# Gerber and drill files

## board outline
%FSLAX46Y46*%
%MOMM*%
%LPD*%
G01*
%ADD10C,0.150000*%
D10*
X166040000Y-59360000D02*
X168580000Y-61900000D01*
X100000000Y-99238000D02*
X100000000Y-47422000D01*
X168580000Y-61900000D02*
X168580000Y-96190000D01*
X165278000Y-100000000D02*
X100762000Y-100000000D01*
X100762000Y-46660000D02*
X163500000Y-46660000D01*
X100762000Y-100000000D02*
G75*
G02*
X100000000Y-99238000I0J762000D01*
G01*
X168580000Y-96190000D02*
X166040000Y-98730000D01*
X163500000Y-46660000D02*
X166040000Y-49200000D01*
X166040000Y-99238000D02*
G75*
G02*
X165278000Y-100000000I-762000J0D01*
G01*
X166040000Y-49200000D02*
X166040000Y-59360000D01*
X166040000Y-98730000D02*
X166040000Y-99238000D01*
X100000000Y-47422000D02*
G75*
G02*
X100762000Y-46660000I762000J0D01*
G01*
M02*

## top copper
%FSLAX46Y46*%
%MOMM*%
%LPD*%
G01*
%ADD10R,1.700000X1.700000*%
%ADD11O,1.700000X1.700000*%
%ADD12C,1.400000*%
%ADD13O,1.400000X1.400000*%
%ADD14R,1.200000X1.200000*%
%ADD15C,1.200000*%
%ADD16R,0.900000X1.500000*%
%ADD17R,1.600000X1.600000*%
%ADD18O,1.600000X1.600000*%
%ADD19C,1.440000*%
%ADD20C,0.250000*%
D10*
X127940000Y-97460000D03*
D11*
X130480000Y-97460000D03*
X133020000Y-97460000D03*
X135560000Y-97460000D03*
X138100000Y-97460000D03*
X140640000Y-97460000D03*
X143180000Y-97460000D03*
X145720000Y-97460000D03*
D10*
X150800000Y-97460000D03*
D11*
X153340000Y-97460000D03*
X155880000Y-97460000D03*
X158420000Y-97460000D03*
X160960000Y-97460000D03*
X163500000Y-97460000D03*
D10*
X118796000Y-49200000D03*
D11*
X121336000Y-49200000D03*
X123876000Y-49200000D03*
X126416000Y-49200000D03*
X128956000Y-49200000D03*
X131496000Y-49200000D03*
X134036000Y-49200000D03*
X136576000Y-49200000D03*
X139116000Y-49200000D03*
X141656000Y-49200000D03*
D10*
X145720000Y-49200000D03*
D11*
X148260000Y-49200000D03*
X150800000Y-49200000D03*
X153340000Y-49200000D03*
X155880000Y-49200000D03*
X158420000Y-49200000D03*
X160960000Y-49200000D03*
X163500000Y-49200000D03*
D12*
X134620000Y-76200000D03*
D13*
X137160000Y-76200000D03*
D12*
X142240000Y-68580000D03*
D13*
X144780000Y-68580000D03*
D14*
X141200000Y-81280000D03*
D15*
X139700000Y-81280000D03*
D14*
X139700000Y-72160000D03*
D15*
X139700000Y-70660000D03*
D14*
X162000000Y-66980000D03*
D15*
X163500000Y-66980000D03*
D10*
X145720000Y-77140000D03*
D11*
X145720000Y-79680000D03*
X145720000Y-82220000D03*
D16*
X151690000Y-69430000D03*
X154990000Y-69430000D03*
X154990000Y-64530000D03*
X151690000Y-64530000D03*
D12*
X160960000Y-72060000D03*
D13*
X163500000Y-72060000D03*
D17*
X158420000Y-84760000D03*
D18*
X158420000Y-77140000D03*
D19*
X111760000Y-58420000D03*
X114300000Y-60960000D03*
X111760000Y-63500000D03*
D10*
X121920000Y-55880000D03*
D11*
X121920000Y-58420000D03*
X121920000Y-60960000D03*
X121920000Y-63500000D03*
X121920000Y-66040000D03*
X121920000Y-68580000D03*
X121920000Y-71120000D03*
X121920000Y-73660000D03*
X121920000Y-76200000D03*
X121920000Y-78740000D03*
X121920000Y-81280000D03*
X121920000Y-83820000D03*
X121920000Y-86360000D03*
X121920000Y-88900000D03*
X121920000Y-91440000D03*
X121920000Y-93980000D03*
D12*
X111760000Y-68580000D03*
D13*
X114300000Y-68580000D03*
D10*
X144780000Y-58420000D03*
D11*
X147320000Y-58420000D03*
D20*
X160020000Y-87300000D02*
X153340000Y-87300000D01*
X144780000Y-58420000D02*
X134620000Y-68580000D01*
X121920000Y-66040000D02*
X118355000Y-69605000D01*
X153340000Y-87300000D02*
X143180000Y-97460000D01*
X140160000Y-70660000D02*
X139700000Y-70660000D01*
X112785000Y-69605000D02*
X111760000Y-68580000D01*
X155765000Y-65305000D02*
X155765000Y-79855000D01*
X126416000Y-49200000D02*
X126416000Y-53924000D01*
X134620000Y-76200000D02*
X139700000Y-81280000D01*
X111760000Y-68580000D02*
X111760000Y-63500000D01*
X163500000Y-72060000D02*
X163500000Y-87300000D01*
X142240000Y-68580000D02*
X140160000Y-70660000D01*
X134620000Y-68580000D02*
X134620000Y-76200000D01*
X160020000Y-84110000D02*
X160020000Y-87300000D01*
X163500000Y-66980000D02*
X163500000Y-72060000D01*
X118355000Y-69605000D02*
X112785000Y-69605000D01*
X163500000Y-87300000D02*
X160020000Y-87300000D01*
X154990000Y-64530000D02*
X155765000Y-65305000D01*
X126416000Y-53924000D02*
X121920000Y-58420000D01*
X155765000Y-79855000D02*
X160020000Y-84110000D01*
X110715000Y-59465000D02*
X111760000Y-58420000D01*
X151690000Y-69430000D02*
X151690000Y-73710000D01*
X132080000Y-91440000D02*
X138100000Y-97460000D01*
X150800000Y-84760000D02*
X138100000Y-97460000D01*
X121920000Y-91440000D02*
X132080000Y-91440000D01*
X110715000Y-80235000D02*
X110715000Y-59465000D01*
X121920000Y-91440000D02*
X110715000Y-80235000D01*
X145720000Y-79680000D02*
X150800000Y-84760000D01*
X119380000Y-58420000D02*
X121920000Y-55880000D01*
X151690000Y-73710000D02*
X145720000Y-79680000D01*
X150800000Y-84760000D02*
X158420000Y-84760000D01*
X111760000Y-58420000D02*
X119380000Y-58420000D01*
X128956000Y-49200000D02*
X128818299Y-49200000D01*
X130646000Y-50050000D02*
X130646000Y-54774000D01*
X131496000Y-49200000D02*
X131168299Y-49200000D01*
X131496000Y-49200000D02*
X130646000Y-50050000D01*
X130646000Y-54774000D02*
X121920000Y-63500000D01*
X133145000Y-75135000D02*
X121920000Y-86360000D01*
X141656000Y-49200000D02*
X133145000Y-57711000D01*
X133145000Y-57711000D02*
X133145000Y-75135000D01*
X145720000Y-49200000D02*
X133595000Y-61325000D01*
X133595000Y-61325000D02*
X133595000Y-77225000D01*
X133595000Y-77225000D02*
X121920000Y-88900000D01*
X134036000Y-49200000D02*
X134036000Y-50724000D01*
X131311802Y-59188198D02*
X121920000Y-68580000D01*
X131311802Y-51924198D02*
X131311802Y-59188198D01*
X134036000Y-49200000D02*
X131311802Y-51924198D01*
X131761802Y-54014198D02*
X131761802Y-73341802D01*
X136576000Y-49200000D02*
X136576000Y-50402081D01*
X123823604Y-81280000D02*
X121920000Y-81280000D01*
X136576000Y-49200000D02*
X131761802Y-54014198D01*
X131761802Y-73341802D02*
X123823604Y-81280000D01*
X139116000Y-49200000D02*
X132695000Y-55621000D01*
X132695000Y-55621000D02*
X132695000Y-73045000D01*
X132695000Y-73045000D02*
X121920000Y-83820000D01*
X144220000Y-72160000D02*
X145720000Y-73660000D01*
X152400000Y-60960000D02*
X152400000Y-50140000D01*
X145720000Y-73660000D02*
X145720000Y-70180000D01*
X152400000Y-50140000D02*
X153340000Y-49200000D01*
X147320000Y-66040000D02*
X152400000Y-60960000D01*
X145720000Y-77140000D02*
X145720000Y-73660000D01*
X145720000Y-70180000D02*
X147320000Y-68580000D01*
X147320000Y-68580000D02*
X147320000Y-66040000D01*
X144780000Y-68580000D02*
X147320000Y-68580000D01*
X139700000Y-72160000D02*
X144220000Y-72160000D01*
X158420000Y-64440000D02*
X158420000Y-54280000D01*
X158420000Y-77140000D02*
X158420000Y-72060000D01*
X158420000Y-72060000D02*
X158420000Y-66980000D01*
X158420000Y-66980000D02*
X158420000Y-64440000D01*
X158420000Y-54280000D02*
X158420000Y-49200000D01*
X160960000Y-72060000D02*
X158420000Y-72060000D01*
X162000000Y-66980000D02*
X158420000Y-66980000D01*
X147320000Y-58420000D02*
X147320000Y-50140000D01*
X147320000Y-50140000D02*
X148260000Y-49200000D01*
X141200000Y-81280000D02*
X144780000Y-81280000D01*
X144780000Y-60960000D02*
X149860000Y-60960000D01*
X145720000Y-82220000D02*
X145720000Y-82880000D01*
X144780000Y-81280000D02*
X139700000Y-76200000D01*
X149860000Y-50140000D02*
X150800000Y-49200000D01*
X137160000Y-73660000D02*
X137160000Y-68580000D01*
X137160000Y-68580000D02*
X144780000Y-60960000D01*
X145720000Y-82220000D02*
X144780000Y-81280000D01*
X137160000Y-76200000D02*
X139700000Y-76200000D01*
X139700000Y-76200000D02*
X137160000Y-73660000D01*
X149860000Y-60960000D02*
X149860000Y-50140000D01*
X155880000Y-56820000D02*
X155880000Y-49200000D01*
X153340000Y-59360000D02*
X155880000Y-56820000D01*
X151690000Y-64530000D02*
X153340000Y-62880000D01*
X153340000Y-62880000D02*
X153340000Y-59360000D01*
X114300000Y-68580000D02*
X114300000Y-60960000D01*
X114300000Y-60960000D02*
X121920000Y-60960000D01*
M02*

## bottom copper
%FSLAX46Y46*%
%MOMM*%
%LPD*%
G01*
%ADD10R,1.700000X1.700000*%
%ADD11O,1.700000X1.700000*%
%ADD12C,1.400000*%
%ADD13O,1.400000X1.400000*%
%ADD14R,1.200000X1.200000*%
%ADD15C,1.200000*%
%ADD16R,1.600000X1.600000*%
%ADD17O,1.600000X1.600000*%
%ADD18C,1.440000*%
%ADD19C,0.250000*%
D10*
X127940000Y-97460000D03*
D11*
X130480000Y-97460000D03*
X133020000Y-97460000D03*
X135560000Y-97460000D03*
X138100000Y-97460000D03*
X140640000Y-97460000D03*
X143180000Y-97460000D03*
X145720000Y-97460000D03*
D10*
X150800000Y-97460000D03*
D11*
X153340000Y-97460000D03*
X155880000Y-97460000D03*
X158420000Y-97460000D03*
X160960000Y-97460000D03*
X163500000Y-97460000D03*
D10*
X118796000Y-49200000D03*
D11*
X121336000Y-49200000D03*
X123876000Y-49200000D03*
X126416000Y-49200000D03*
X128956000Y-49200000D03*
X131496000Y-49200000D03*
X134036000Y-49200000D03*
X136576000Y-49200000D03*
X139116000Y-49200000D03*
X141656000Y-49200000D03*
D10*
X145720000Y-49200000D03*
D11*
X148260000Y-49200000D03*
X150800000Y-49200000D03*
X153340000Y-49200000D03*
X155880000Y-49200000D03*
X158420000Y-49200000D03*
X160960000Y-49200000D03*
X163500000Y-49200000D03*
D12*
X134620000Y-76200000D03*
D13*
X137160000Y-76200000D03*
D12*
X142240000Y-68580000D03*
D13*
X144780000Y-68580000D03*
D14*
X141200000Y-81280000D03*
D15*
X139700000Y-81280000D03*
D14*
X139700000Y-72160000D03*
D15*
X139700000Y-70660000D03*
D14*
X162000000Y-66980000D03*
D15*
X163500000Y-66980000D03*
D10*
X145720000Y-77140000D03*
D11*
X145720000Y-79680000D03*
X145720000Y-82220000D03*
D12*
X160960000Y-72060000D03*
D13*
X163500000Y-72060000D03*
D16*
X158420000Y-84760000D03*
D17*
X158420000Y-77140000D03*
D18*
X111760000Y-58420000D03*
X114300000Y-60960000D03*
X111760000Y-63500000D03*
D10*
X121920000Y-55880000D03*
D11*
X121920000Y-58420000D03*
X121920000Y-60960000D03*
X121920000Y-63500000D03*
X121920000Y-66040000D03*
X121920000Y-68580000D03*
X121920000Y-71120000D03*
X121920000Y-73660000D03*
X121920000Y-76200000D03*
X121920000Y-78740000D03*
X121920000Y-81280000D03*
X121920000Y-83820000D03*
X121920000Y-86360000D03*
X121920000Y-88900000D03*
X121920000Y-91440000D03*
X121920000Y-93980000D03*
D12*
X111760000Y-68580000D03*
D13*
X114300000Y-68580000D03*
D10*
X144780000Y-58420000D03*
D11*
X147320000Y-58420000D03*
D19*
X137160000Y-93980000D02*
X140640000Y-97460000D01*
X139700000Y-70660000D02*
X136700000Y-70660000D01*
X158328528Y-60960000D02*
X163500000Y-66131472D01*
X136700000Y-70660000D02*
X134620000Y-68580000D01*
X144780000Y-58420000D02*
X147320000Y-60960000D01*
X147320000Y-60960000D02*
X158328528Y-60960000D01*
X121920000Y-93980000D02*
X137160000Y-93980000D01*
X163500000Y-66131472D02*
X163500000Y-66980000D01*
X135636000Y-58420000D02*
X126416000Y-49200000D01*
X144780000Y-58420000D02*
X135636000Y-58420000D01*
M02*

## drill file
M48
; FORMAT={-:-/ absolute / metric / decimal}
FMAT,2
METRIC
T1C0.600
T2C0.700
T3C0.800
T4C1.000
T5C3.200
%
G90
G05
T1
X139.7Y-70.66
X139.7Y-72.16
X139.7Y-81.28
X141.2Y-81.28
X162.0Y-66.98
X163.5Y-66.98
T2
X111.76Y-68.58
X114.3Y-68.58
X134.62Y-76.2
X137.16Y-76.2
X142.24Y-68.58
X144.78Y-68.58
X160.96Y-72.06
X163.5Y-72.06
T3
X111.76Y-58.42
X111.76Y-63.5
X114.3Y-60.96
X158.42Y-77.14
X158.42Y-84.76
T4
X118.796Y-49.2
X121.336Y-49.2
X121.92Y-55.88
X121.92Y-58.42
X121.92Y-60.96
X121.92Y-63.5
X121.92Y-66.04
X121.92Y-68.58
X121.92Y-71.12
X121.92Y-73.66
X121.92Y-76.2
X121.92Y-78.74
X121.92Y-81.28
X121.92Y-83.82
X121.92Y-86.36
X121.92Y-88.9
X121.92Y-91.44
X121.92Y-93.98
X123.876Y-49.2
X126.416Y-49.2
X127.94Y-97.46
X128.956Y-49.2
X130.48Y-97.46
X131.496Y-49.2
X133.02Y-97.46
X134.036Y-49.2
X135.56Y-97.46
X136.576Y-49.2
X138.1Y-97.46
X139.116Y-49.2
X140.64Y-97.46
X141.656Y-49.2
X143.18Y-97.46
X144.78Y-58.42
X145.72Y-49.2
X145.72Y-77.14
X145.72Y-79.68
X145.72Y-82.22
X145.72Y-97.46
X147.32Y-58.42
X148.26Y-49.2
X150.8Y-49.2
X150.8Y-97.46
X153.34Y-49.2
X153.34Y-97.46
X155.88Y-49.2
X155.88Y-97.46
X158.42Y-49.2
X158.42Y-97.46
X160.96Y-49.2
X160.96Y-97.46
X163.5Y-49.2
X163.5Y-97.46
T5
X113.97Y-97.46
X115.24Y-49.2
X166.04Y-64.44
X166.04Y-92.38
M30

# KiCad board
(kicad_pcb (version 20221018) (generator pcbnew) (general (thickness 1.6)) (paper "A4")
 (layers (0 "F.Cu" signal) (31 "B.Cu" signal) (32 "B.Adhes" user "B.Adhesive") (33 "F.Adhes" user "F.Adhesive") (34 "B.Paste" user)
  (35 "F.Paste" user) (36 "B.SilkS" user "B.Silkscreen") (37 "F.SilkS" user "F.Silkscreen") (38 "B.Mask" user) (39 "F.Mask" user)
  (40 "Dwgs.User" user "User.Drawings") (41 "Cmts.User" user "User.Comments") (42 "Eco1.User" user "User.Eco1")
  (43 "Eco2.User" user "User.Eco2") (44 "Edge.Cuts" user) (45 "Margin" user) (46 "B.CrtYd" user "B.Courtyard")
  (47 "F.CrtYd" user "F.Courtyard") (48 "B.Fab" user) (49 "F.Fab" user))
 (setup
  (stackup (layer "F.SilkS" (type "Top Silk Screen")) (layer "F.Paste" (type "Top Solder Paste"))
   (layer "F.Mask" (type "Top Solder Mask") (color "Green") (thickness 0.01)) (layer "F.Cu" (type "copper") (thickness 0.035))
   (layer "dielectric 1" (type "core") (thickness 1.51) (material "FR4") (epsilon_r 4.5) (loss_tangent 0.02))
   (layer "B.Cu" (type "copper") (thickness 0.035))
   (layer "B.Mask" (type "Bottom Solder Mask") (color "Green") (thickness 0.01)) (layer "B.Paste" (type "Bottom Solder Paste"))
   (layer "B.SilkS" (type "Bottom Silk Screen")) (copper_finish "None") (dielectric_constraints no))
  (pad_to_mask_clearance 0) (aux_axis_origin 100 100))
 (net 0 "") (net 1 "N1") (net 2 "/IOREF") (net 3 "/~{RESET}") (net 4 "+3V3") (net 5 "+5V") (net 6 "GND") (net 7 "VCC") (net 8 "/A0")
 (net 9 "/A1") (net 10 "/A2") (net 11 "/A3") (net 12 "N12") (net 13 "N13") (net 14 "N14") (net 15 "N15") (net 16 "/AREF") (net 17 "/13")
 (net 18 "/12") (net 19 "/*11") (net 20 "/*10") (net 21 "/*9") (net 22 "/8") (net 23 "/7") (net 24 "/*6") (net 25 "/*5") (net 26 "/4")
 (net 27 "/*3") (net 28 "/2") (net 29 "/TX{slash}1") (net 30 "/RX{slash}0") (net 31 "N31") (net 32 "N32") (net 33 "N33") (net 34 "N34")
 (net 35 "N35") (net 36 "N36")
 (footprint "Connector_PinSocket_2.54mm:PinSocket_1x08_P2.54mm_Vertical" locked (layer "F.Cu") (at 127.94 97.46 90)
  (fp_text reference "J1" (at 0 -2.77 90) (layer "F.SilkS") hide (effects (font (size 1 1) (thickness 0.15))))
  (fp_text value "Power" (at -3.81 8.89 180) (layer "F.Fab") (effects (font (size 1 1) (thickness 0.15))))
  (pad "1" thru_hole rect locked (at 0 0 90) (size 1.7 1.7) (drill 1) (layers "*.Cu" "*.Mask") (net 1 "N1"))
  (pad "2" thru_hole oval locked (at 0 2.54 90) (size 1.7 1.7) (drill 1) (layers "*.Cu" "*.Mask") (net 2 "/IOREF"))
  (pad "3" thru_hole oval locked (at 0 5.08 90) (size 1.7 1.7) (drill 1) (layers "*.Cu" "*.Mask") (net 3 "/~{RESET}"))
  (pad "4" thru_hole oval locked (at 0 7.62 90) (size 1.7 1.7) (drill 1) (layers "*.Cu" "*.Mask") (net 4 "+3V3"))
  (pad "5" thru_hole oval locked (at 0 10.16 90) (size 1.7 1.7) (drill 1) (layers "*.Cu" "*.Mask") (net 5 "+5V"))
  (pad "6" thru_hole oval locked (at 0 12.7 90) (size 1.7 1.7) (drill 1) (layers "*.Cu" "*.Mask") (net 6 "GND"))
  (pad "7" thru_hole oval locked (at 0 15.24 90) (size 1.7 1.7) (drill 1) (layers "*.Cu" "*.Mask") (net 6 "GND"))
  (pad "8" thru_hole oval locked (at 0 17.78 90) (size 1.7 1.7) (drill 1) (layers "*.Cu" "*.Mask") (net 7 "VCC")))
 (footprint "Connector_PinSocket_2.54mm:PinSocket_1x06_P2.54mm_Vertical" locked (layer "F.Cu") (at 150.8 97.46 90)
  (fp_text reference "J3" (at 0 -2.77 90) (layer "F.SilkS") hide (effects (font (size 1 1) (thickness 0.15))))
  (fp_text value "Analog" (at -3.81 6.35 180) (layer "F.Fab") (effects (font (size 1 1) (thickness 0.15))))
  (pad "1" thru_hole rect locked (at 0 0 90) (size 1.7 1.7) (drill 1) (layers "*.Cu" "*.Mask") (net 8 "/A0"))
  (pad "2" thru_hole oval locked (at 0 2.54 90) (size 1.7 1.7) (drill 1) (layers "*.Cu" "*.Mask") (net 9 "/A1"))
  (pad "3" thru_hole oval locked (at 0 5.08 90) (size 1.7 1.7) (drill 1) (layers "*.Cu" "*.Mask") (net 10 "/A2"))
  (pad "4" thru_hole oval locked (at 0 7.62 90) (size 1.7 1.7) (drill 1) (layers "*.Cu" "*.Mask") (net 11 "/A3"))
  (pad "5" thru_hole oval locked (at 0 10.16 90) (size 1.7 1.7) (drill 1) (layers "*.Cu" "*.Mask") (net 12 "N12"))
  (pad "6" thru_hole oval locked (at 0 12.7 90) (size 1.7 1.7) (drill 1) (layers "*.Cu" "*.Mask") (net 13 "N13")))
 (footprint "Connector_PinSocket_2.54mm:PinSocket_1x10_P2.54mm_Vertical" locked (layer "F.Cu") (at 118.796 49.2 90)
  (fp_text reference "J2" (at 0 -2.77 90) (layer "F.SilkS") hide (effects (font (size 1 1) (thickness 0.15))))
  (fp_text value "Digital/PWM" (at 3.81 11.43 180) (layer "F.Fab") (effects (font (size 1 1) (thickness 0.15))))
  (pad "1" thru_hole rect locked (at 0 0 90) (size 1.7 1.7) (drill 1) (layers "*.Cu" "*.Mask") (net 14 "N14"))
  (pad "2" thru_hole oval locked (at 0 2.54 90) (size 1.7 1.7) (drill 1) (layers "*.Cu" "*.Mask") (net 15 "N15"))
  (pad "3" thru_hole oval locked (at 0 5.08 90) (size 1.7 1.7) (drill 1) (layers "*.Cu" "*.Mask") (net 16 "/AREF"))
  (pad "4" thru_hole oval locked (at 0 7.62 90) (size 1.7 1.7) (drill 1) (layers "*.Cu" "*.Mask") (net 6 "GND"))
  (pad "5" thru_hole oval locked (at 0 10.16 90) (size 1.7 1.7) (drill 1) (layers "*.Cu" "*.Mask") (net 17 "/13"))
  (pad "6" thru_hole oval locked (at 0 12.7 90) (size 1.7 1.7) (drill 1) (layers "*.Cu" "*.Mask") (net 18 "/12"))
  (pad "7" thru_hole oval locked (at 0 15.24 90) (size 1.7 1.7) (drill 1) (layers "*.Cu" "*.Mask") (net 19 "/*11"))
  (pad "8" thru_hole oval locked (at 0 17.78 90) (size 1.7 1.7) (drill 1) (layers "*.Cu" "*.Mask") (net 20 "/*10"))
  (pad "9" thru_hole oval locked (at 0 20.32 90) (size 1.7 1.7) (drill 1) (layers "*.Cu" "*.Mask") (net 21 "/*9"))
  (pad "10" thru_hole oval locked (at 0 22.86 90) (size 1.7 1.7) (drill 1) (layers "*.Cu" "*.Mask") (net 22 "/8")))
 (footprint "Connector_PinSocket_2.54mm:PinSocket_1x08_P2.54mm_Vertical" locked (layer "F.Cu") (at 145.72 49.2 90)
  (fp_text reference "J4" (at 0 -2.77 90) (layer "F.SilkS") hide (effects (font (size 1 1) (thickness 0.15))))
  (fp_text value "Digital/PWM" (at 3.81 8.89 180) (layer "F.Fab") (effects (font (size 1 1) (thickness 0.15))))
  (pad "1" thru_hole rect locked (at 0 0 90) (size 1.7 1.7) (drill 1) (layers "*.Cu" "*.Mask") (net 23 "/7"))
  (pad "2" thru_hole oval locked (at 0 2.54 90) (size 1.7 1.7) (drill 1) (layers "*.Cu" "*.Mask") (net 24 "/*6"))
  (pad "3" thru_hole oval locked (at 0 5.08 90) (size 1.7 1.7) (drill 1) (layers "*.Cu" "*.Mask") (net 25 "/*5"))
  (pad "4" thru_hole oval locked (at 0 7.62 90) (size 1.7 1.7) (drill 1) (layers "*.Cu" "*.Mask") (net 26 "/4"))
  (pad "5" thru_hole oval locked (at 0 10.16 90) (size 1.7 1.7) (drill 1) (layers "*.Cu" "*.Mask") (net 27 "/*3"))
  (pad "6" thru_hole oval locked (at 0 12.7 90) (size 1.7 1.7) (drill 1) (layers "*.Cu" "*.Mask") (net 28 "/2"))
  (pad "7" thru_hole oval locked (at 0 15.24 90) (size 1.7 1.7) (drill 1) (layers "*.Cu" "*.Mask") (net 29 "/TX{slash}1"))
  (pad "8" thru_hole oval locked (at 0 17.78 90) (size 1.7 1.7) (drill 1) (layers "*.Cu" "*.Mask") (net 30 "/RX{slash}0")))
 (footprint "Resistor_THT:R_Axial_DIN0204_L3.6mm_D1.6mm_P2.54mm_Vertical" (layer "F.Cu") (at 134.62 76.2)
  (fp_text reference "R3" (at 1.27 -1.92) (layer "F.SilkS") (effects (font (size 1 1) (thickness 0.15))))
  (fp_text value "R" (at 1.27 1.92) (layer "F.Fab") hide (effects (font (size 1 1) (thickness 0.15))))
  (pad "1" thru_hole circle (at 0 0) (size 1.4 1.4) (drill 0.7) (layers "*.Cu" "*.Mask") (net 6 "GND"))
  (pad "2" thru_hole oval (at 2.54 0) (size 1.4 1.4) (drill 0.7) (layers "*.Cu" "*.Mask") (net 25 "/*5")))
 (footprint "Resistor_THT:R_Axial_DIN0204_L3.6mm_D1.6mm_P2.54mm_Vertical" (layer "F.Cu") (at 142.24 68.58)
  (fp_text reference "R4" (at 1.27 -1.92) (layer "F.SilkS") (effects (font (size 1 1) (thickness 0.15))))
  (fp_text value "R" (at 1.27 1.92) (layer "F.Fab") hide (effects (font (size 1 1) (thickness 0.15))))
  (pad "1" thru_hole circle (at 0 0) (size 1.4 1.4) (drill 0.7) (layers "*.Cu" "*.Mask") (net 6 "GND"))
  (pad "2" thru_hole oval (at 2.54 0) (size 1.4 1.4) (drill 0.7) (layers "*.Cu" "*.Mask") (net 26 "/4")))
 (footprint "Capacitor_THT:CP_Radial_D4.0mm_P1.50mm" (layer "F.Cu") (at 141.2 81.28 180)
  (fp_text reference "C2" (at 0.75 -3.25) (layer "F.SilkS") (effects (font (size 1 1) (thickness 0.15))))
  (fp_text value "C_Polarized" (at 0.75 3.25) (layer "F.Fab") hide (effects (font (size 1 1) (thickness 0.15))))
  (pad "1" thru_hole rect (at 0 0 180) (size 1.2 1.2) (drill 0.6) (layers "*.Cu" "*.Mask") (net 25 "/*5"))
  (pad "2" thru_hole circle (at 1.5 0 180) (size 1.2 1.2) (drill 0.6) (layers "*.Cu" "*.Mask") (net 6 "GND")))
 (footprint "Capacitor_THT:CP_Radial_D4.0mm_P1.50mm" (layer "F.Cu") (at 139.7 72.16 90)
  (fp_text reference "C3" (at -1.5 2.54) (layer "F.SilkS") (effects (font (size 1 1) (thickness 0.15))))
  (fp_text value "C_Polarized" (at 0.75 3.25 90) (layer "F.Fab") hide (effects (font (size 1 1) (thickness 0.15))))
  (pad "1" thru_hole rect (at 0 0 90) (size 1.2 1.2) (drill 0.6) (layers "*.Cu" "*.Mask") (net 26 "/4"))
  (pad "2" thru_hole circle (at 1.5 0 90) (size 1.2 1.2) (drill 0.6) (layers "*.Cu" "*.Mask") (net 6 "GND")))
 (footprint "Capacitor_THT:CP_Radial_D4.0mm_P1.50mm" (layer "F.Cu") (at 162 66.98)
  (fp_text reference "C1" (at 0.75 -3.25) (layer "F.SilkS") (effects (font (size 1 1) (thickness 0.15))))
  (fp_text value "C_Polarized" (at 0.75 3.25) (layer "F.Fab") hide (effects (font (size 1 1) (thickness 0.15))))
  (pad "1" thru_hole rect (at 0 0) (size 1.2 1.2) (drill 0.6) (layers "*.Cu" "*.Mask") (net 28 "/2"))
  (pad "2" thru_hole circle (at 1.5 0) (size 1.2 1.2) (drill 0.6) (layers "*.Cu" "*.Mask") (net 6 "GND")))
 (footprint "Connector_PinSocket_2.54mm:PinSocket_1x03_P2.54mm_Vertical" (layer "F.Cu") (at 145.72 77.14)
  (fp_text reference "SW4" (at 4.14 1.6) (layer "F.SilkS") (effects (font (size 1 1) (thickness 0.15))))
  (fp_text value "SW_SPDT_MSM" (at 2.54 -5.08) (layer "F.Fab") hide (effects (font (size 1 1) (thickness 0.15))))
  (pad "1" thru_hole rect (at 0 0) (size 1.7 1.7) (drill 1) (layers "*.Cu" "*.Mask") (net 26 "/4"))
  (pad "2" thru_hole oval (at 0 2.54) (size 1.7 1.7) (drill 1) (layers "*.Cu" "*.Mask") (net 5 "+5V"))
  (pad "3" thru_hole oval (at 0 5.08) (size 1.7 1.7) (drill 1) (layers "*.Cu" "*.Mask") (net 25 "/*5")))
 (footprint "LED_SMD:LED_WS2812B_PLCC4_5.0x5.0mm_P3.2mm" (layer "F.Cu") (at 153.34 66.98 90)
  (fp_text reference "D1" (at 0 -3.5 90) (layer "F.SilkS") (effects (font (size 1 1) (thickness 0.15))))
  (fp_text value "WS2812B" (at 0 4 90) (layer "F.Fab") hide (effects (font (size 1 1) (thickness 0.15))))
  (pad "1" smd rect (at -2.45 -1.65 90) (size 1.5 0.9) (layers "F.Cu" "F.Paste" "F.Mask") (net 5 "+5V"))
  (pad "2" smd rect (at -2.45 1.65 90) (size 1.5 0.9) (layers "F.Cu" "F.Paste" "F.Mask") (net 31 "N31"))
  (pad "3" smd rect (at 2.45 1.65 90) (size 1.5 0.9) (layers "F.Cu" "F.Paste" "F.Mask") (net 6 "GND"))
  (pad "4" smd rect (at 2.45 -1.65 90) (size 1.5 0.9) (layers "F.Cu" "F.Paste" "F.Mask") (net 27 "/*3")))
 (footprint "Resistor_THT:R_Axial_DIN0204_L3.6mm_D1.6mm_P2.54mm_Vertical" (layer "F.Cu") (at 160.96 72.06)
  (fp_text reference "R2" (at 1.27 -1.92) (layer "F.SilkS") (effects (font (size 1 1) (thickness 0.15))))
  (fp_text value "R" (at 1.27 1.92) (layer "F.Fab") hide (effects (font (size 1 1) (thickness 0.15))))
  (pad "1" thru_hole circle (at 0 0) (size 1.4 1.4) (drill 0.7) (layers "*.Cu" "*.Mask") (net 28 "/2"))
  (pad "2" thru_hole oval (at 2.54 0) (size 1.4 1.4) (drill 0.7) (layers "*.Cu" "*.Mask") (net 6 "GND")))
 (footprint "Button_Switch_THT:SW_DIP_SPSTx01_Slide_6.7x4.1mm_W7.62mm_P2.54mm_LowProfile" (layer "F.Cu") (at 158.42 84.76 90)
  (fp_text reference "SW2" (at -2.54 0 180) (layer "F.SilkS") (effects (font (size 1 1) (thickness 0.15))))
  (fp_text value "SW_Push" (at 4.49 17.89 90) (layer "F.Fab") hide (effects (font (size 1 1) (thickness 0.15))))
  (pad "1" thru_hole rect (at 0 0 90) (size 1.6 1.6) (drill 0.8) (layers "*.Cu" "*.Mask") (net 5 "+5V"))
  (pad "2" thru_hole oval (at 7.62 0 90) (size 1.6 1.6) (drill 0.8) (layers "*.Cu" "*.Mask") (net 28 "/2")))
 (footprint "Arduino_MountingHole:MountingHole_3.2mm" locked (layer "F.Cu") (at 115.24 49.2)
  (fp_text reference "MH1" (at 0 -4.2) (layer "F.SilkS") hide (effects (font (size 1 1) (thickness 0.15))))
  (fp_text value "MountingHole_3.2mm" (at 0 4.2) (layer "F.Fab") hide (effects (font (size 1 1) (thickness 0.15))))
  (pad "" np_thru_hole circle locked (at 0 0) (size 3.2 3.2) (drill 3.2) (layers "*.Cu" "*.Mask")))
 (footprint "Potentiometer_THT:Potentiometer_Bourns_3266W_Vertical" (layer "F.Cu") (at 111.76 58.42 90)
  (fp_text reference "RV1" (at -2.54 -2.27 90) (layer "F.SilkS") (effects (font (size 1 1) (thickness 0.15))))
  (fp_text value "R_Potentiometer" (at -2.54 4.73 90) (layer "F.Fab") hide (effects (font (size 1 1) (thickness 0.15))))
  (pad "1" thru_hole circle (at 0 0 90) (size 1.44 1.44) (drill 0.8) (layers "*.Cu" "*.Mask") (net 5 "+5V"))
  (pad "2" thru_hole circle (at -2.54 2.54 90) (size 1.44 1.44) (drill 0.8) (layers "*.Cu" "*.Mask") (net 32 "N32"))
  (pad "3" thru_hole circle (at -5.08 0 90) (size 1.44 1.44) (drill 0.8) (layers "*.Cu" "*.Mask") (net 6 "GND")))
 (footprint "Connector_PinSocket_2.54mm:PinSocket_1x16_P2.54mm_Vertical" (layer "F.Cu") (at 121.92 55.88)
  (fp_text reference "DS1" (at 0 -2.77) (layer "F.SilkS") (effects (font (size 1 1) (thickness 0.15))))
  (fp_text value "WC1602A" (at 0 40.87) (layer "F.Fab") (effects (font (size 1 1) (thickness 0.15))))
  (pad "1" thru_hole rect (at 0 0) (size 1.7 1.7) (drill 1) (layers "*.Cu" "*.Mask") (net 5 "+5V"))
  (pad "2" thru_hole oval (at 0 2.54) (size 1.7 1.7) (drill 1) (layers "*.Cu" "*.Mask") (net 6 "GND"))
  (pad "3" thru_hole oval (at 0 5.08) (size 1.7 1.7) (drill 1) (layers "*.Cu" "*.Mask") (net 32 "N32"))
  (pad "4" thru_hole oval (at 0 7.62) (size 1.7 1.7) (drill 1) (layers "*.Cu" "*.Mask") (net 18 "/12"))
  (pad "5" thru_hole oval (at 0 10.16) (size 1.7 1.7) (drill 1) (layers "*.Cu" "*.Mask") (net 6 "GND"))
  (pad "6" thru_hole oval (at 0 12.7) (size 1.7 1.7) (drill 1) (layers "*.Cu" "*.Mask") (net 19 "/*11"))
  (pad "7" thru_hole oval (at 0 15.24) (size 1.7 1.7) (drill 1) (layers "*.Cu" "*.Mask") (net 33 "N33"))
  (pad "8" thru_hole oval (at 0 17.78) (size 1.7 1.7) (drill 1) (layers "*.Cu" "*.Mask") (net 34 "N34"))
  (pad "9" thru_hole oval (at 0 20.32) (size 1.7 1.7) (drill 1) (layers "*.Cu" "*.Mask") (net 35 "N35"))
  (pad "10" thru_hole oval (at 0 22.86) (size 1.7 1.7) (drill 1) (layers "*.Cu" "*.Mask") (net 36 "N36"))
  (pad "11" thru_hole oval (at 0 25.4) (size 1.7 1.7) (drill 1) (layers "*.Cu" "*.Mask") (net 20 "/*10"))
  (pad "12" thru_hole oval (at 0 27.94) (size 1.7 1.7) (drill 1) (layers "*.Cu" "*.Mask") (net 21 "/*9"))
  (pad "13" thru_hole oval (at 0 30.48) (size 1.7 1.7) (drill 1) (layers "*.Cu" "*.Mask") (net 22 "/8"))
  (pad "14" thru_hole oval (at 0 33.02) (size 1.7 1.7) (drill 1) (layers "*.Cu" "*.Mask") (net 23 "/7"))
  (pad "15" thru_hole oval (at 0 35.56) (size 1.7 1.7) (drill 1) (layers "*.Cu" "*.Mask") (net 5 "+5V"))
  (pad "16" thru_hole oval (at 0 38.1) (size 1.7 1.7) (drill 1) (layers "*.Cu" "*.Mask") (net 6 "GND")))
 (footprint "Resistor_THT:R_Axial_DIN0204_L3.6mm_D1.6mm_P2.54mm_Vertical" (layer "F.Cu") (at 111.76 68.58)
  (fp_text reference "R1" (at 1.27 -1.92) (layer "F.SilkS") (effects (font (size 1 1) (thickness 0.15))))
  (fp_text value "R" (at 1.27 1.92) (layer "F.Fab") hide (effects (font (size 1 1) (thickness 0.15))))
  (pad "1" thru_hole circle (at 0 0) (size 1.4 1.4) (drill 0.7) (layers "*.Cu" "*.Mask") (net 6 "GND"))
  (pad "2" thru_hole oval (at 2.54 0) (size 1.4 1.4) (drill 0.7) (layers "*.Cu" "*.Mask") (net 32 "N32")))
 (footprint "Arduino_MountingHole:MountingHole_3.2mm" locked (layer "F.Cu") (at 113.97 97.46)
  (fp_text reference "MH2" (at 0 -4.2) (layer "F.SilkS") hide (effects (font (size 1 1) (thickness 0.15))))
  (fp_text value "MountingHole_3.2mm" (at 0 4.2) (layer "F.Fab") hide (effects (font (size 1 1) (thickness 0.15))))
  (pad "" np_thru_hole circle locked (at 0 0) (size 3.2 3.2) (drill 3.2) (layers "*.Cu" "*.Mask")))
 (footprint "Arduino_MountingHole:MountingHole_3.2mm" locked (layer "F.Cu") (at 166.04 64.44)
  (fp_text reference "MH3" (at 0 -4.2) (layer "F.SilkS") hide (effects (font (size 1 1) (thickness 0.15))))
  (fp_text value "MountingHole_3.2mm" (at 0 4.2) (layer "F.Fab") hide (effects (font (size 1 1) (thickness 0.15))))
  (pad "" np_thru_hole circle locked (at 0 0) (size 3.2 3.2) (drill 3.2) (layers "*.Cu" "*.Mask")))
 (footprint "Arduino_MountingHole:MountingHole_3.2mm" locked (layer "F.Cu") (at 166.04 92.38)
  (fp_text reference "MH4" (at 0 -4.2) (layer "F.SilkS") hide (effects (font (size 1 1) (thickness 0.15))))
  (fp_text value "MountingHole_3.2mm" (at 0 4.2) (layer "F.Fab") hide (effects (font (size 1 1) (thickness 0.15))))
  (pad "" np_thru_hole circle locked (at 0 0) (size 3.2 3.2) (drill 3.2) (layers "*.Cu" "*.Mask")))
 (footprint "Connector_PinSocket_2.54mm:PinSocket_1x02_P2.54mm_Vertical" (layer "F.Cu") (at 144.78 58.42 90)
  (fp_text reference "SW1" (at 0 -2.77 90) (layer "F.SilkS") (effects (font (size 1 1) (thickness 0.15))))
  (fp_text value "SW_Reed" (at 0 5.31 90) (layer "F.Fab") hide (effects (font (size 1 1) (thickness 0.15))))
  (pad "1" thru_hole rect (at 0 0 90) (size 1.7 1.7) (drill 1) (layers "*.Cu" "*.Mask") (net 6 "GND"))
  (pad "2" thru_hole oval (at 0 2.54 90) (size 1.7 1.7) (drill 1) (layers "*.Cu" "*.Mask") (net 24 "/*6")))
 (gr_line (start 166.04 59.36) (end 168.58 61.9) (stroke (width 0.15) (type solid)) (layer "Edge.Cuts"))
 (gr_line (start 100 99.238) (end 100 47.422) (stroke (width 0.15) (type solid)) (layer "Edge.Cuts"))
 (gr_line (start 168.58 61.9) (end 168.58 96.19) (stroke (width 0.15) (type solid)) (layer "Edge.Cuts"))
 (gr_line (start 165.278 100) (end 100.762 100) (stroke (width 0.15) (type solid)) (layer "Edge.Cuts"))
 (gr_line (start 100.762 46.66) (end 163.5 46.66) (stroke (width 0.15) (type solid)) (layer "Edge.Cuts"))
 (gr_arc (start 100.762 100) (mid 100.223185 99.776815) (end 100 99.238) (stroke (width 0.15) (type solid)) (layer "Edge.Cuts"))
 (gr_line (start 168.58 96.19) (end 166.04 98.73) (stroke (width 0.15) (type solid)) (layer "Edge.Cuts"))
 (gr_line (start 163.5 46.66) (end 166.04 49.2) (stroke (width 0.15) (type solid)) (layer "Edge.Cuts"))
 (gr_arc (start 166.04 99.238) (mid 165.816815 99.776815) (end 165.278 100) (stroke (width 0.15) (type solid)) (layer "Edge.Cuts"))
 (gr_line (start 166.04 49.2) (end 166.04 59.36) (stroke (width 0.15) (type solid)) (layer "Edge.Cuts"))
 (gr_line (start 166.04 98.73) (end 166.04 99.238) (stroke (width 0.15) (type solid)) (layer "Edge.Cuts"))
 (gr_arc (start 100 47.422) (mid 100.223185 46.883185) (end 100.762 46.66) (stroke (width 0.15) (type solid)) (layer "Edge.Cuts"))
 (segment (start 160.02 87.3) (end 153.34 87.3) (width 0.25) (layer "F.Cu") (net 6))
 (segment (start 144.78 58.42) (end 134.62 68.58) (width 0.25) (layer "F.Cu") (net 6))
 (segment (start 121.92 66.04) (end 118.355 69.605) (width 0.25) (layer "F.Cu") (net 6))
 (segment (start 153.34 87.3) (end 143.18 97.46) (width 0.25) (layer "F.Cu") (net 6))
 (segment (start 140.16 70.66) (end 139.7 70.66) (width 0.25) (layer "F.Cu") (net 6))
 (segment (start 112.785 69.605) (end 111.76 68.58) (width 0.25) (layer "F.Cu") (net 6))
 (segment (start 155.765 65.305) (end 155.765 79.855) (width 0.25) (layer "F.Cu") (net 6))
 (segment (start 126.416 49.2) (end 126.416 53.924) (width 0.25) (layer "F.Cu") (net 6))
 (segment (start 134.62 76.2) (end 139.7 81.28) (width 0.25) (layer "F.Cu") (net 6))
 (segment (start 111.76 68.58) (end 111.76 63.5) (width 0.25) (layer "F.Cu") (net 6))
 (segment (start 163.5 72.06) (end 163.5 87.3) (width 0.25) (layer "F.Cu") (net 6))
 (segment (start 142.24 68.58) (end 140.16 70.66) (width 0.25) (layer "F.Cu") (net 6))
 (segment (start 134.62 68.58) (end 134.62 76.2) (width 0.25) (layer "F.Cu") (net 6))
 (segment (start 160.02 84.11) (end 160.02 87.3) (width 0.25) (layer "F.Cu") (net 6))
 (segment (start 163.5 66.98) (end 163.5 72.06) (width 0.25) (layer "F.Cu") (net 6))
 (segment (start 118.355 69.605) (end 112.785 69.605) (width 0.25) (layer "F.Cu") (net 6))
 (segment (start 163.5 87.3) (end 160.02 87.3) (width 0.25) (layer "F.Cu") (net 6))
 (segment (start 154.99 64.53) (end 155.765 65.305) (width 0.25) (layer "F.Cu") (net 6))
 (segment (start 126.416 53.924) (end 121.92 58.42) (width 0.25) (layer "F.Cu") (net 6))
 (segment (start 155.765 79.855) (end 160.02 84.11) (width 0.25) (layer "F.Cu") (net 6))
 (segment (start 137.16 93.98) (end 140.64 97.46) (width 0.25) (layer "B.Cu") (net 6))
 (segment (start 139.7 70.66) (end 136.7 70.66) (width 0.25) (layer "B.Cu") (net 6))
 (segment (start 158.328528 60.96) (end 163.5 66.131472) (width 0.25) (layer "B.Cu") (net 6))
 (segment (start 136.7 70.66) (end 134.62 68.58) (width 0.25) (layer "B.Cu") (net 6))
 (segment (start 144.78 58.42) (end 147.32 60.96) (width 0.25) (layer "B.Cu") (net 6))
 (segment (start 147.32 60.96) (end 158.328528 60.96) (width 0.25) (layer "B.Cu") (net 6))
 (segment (start 121.92 93.98) (end 137.16 93.98) (width 0.25) (layer "B.Cu") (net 6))
 (segment (start 163.5 66.131472) (end 163.5 66.98) (width 0.25) (layer "B.Cu") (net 6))
 (segment (start 135.636 58.42) (end 126.416 49.2) (width 0.25) (layer "B.Cu") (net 6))
 (segment (start 144.78 58.42) (end 135.636 58.42) (width 0.25) (layer "B.Cu") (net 6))
 (segment (start 110.715 59.465) (end 111.76 58.42) (width 0.25) (layer "F.Cu") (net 5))
 (segment (start 151.69 69.43) (end 151.69 73.71) (width 0.25) (layer "F.Cu") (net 5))
 (segment (start 132.08 91.44) (end 138.1 97.46) (width 0.25) (layer "F.Cu") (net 5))
 (segment (start 150.8 84.76) (end 138.1 97.46) (width 0.25) (layer "F.Cu") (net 5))
 (segment (start 121.92 91.44) (end 132.08 91.44) (width 0.25) (layer "F.Cu") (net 5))
 (segment (start 110.715 80.235) (end 110.715 59.465) (width 0.25) (layer "F.Cu") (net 5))
 (segment (start 121.92 91.44) (end 110.715 80.235) (width 0.25) (layer "F.Cu") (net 5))
 (segment (start 145.72 79.68) (end 150.8 84.76) (width 0.25) (layer "F.Cu") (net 5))
 (segment (start 119.38 58.42) (end 121.92 55.88) (width 0.25) (layer "F.Cu") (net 5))
 (segment (start 151.69 73.71) (end 145.72 79.68) (width 0.25) (layer "F.Cu") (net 5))
 (segment (start 150.8 84.76) (end 158.42 84.76) (width 0.25) (layer "F.Cu") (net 5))
 (segment (start 111.76 58.42) (end 119.38 58.42) (width 0.25) (layer "F.Cu") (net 5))
 (segment (start 128.956 49.2) (end 128.818299 49.2) (width 0.25) (layer "F.Cu") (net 17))
 (segment (start 130.646 50.05) (end 130.646 54.774) (width 0.25) (layer "F.Cu") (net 18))
 (segment (start 131.496 49.2) (end 131.168299 49.2) (width 0.25) (layer "F.Cu") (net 18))
 (segment (start 131.496 49.2) (end 130.646 50.05) (width 0.25) (layer "F.Cu") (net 18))
 (segment (start 130.646 54.774) (end 121.92 63.5) (width 0.25) (layer "F.Cu") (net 18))
 (segment (start 133.145 75.135) (end 121.92 86.36) (width 0.25) (layer "F.Cu") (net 22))
 (segment (start 141.656 49.2) (end 133.145 57.711) (width 0.25) (layer "F.Cu") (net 22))
 (segment (start 133.145 57.711) (end 133.145 75.135) (width 0.25) (layer "F.Cu") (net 22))
 (segment (start 145.72 49.2) (end 133.595 61.325) (width 0.25) (layer "F.Cu") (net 23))
 (segment (start 133.595 61.325) (end 133.595 77.225) (width 0.25) (layer "F.Cu") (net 23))
 (segment (start 133.595 77.225) (end 121.92 88.9) (width 0.25) (layer "F.Cu") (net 23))
 (segment (start 134.036 49.2) (end 134.036 50.724) (width 0.25) (layer "F.Cu") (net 19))
 (segment (start 131.311802 59.188198) (end 121.92 68.58) (width 0.25) (layer "F.Cu") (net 19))
 (segment (start 131.311802 51.924198) (end 131.311802 59.188198) (width 0.25) (layer "F.Cu") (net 19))
 (segment (start 134.036 49.2) (end 131.311802 51.924198) (width 0.25) (layer "F.Cu") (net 19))
 (segment (start 131.761802 54.014198) (end 131.761802 73.341802) (width 0.25) (layer "F.Cu") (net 20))
 (segment (start 136.576 49.2) (end 136.576 50.402081) (width 0.25) (layer "F.Cu") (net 20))
 (segment (start 123.823604 81.28) (end 121.92 81.28) (width 0.25) (layer "F.Cu") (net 20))
 (segment (start 136.576 49.2) (end 131.761802 54.014198) (width 0.25) (layer "F.Cu") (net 20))
 (segment (start 131.761802 73.341802) (end 123.823604 81.28) (width 0.25) (layer "F.Cu") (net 20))
 (segment (start 139.116 49.2) (end 132.695 55.621) (width 0.25) (layer "F.Cu") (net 21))
 (segment (start 132.695 55.621) (end 132.695 73.045) (width 0.25) (layer "F.Cu") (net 21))
 (segment (start 132.695 73.045) (end 121.92 83.82) (width 0.25) (layer "F.Cu") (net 21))
 (segment (start 144.22 72.16) (end 145.72 73.66) (width 0.25) (layer "F.Cu") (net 26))
 (segment (start 152.4 60.96) (end 152.4 50.14) (width 0.25) (layer "F.Cu") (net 26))
 (segment (start 145.72 73.66) (end 145.72 70.18) (width 0.25) (layer "F.Cu") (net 26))
 (segment (start 152.4 50.14) (end 153.34 49.2) (width 0.25) (layer "F.Cu") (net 26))
 (segment (start 147.32 66.04) (end 152.4 60.96) (width 0.25) (layer "F.Cu") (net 26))
 (segment (start 145.72 77.14) (end 145.72 73.66) (width 0.25) (layer "F.Cu") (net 26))
 (segment (start 145.72 70.18) (end 147.32 68.58) (width 0.25) (layer "F.Cu") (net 26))
 (segment (start 147.32 68.58) (end 147.32 66.04) (width 0.25) (layer "F.Cu") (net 26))
 (segment (start 144.78 68.58) (end 147.32 68.58) (width 0.25) (layer "F.Cu") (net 26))
 (segment (start 139.7 72.16) (end 144.22 72.16) (width 0.25) (layer "F.Cu") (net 26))
 (segment (start 158.42 64.44) (end 158.42 54.28) (width 0.25) (layer "F.Cu") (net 28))
 (segment (start 158.42 77.14) (end 158.42 72.06) (width 0.25) (layer "F.Cu") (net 28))
 (segment (start 158.42 72.06) (end 158.42 66.98) (width 0.25) (layer "F.Cu") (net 28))
 (segment (start 158.42 66.98) (end 158.42 64.44) (width 0.25) (layer "F.Cu") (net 28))
 (segment (start 158.42 54.28) (end 158.42 49.2) (width 0.25) (layer "F.Cu") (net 28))
 (segment (start 160.96 72.06) (end 158.42 72.06) (width 0.25) (layer "F.Cu") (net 28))
 (segment (start 162 66.98) (end 158.42 66.98) (width 0.25) (layer "F.Cu") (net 28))
 (segment (start 147.32 58.42) (end 147.32 50.14) (width 0.25) (layer "F.Cu") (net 24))
 (segment (start 147.32 50.14) (end 148.26 49.2) (width 0.25) (layer "F.Cu") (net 24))
 (segment (start 141.2 81.28) (end 144.78 81.28) (width 0.25) (layer "F.Cu") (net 25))
 (segment (start 144.78 60.96) (end 149.86 60.96) (width 0.25) (layer "F.Cu") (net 25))
 (segment (start 145.72 82.22) (end 145.72 82.88) (width 0.25) (layer "F.Cu") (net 25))
 (segment (start 144.78 81.28) (end 139.7 76.2) (width 0.25) (layer "F.Cu") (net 25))
 (segment (start 149.86 50.14) (end 150.8 49.2) (width 0.25) (layer "F.Cu") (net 25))
 (segment (start 137.16 73.66) (end 137.16 68.58) (width 0.25) (layer "F.Cu") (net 25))
 (segment (start 137.16 68.58) (end 144.78 60.96) (width 0.25) (layer "F.Cu") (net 25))
 (segment (start 145.72 82.22) (end 144.78 81.28) (width 0.25) (layer "F.Cu") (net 25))
 (segment (start 137.16 76.2) (end 139.7 76.2) (width 0.25) (layer "F.Cu") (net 25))
 (segment (start 139.7 76.2) (end 137.16 73.66) (width 0.25) (layer "F.Cu") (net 25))
 (segment (start 149.86 60.96) (end 149.86 50.14) (width 0.25) (layer "F.Cu") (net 25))
 (segment (start 155.88 56.82) (end 155.88 49.2) (width 0.25) (layer "F.Cu") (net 27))
 (segment (start 153.34 59.36) (end 155.88 56.82) (width 0.25) (layer "F.Cu") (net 27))
 (segment (start 151.69 64.53) (end 153.34 62.88) (width 0.25) (layer "F.Cu") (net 27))
 (segment (start 153.34 62.88) (end 153.34 59.36) (width 0.25) (layer "F.Cu") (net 27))
 (segment (start 114.3 68.58) (end 114.3 60.96) (width 0.25) (layer "F.Cu") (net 32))
 (segment (start 114.3 60.96) (end 121.92 60.96) (width 0.25) (layer "F.Cu") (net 32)))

